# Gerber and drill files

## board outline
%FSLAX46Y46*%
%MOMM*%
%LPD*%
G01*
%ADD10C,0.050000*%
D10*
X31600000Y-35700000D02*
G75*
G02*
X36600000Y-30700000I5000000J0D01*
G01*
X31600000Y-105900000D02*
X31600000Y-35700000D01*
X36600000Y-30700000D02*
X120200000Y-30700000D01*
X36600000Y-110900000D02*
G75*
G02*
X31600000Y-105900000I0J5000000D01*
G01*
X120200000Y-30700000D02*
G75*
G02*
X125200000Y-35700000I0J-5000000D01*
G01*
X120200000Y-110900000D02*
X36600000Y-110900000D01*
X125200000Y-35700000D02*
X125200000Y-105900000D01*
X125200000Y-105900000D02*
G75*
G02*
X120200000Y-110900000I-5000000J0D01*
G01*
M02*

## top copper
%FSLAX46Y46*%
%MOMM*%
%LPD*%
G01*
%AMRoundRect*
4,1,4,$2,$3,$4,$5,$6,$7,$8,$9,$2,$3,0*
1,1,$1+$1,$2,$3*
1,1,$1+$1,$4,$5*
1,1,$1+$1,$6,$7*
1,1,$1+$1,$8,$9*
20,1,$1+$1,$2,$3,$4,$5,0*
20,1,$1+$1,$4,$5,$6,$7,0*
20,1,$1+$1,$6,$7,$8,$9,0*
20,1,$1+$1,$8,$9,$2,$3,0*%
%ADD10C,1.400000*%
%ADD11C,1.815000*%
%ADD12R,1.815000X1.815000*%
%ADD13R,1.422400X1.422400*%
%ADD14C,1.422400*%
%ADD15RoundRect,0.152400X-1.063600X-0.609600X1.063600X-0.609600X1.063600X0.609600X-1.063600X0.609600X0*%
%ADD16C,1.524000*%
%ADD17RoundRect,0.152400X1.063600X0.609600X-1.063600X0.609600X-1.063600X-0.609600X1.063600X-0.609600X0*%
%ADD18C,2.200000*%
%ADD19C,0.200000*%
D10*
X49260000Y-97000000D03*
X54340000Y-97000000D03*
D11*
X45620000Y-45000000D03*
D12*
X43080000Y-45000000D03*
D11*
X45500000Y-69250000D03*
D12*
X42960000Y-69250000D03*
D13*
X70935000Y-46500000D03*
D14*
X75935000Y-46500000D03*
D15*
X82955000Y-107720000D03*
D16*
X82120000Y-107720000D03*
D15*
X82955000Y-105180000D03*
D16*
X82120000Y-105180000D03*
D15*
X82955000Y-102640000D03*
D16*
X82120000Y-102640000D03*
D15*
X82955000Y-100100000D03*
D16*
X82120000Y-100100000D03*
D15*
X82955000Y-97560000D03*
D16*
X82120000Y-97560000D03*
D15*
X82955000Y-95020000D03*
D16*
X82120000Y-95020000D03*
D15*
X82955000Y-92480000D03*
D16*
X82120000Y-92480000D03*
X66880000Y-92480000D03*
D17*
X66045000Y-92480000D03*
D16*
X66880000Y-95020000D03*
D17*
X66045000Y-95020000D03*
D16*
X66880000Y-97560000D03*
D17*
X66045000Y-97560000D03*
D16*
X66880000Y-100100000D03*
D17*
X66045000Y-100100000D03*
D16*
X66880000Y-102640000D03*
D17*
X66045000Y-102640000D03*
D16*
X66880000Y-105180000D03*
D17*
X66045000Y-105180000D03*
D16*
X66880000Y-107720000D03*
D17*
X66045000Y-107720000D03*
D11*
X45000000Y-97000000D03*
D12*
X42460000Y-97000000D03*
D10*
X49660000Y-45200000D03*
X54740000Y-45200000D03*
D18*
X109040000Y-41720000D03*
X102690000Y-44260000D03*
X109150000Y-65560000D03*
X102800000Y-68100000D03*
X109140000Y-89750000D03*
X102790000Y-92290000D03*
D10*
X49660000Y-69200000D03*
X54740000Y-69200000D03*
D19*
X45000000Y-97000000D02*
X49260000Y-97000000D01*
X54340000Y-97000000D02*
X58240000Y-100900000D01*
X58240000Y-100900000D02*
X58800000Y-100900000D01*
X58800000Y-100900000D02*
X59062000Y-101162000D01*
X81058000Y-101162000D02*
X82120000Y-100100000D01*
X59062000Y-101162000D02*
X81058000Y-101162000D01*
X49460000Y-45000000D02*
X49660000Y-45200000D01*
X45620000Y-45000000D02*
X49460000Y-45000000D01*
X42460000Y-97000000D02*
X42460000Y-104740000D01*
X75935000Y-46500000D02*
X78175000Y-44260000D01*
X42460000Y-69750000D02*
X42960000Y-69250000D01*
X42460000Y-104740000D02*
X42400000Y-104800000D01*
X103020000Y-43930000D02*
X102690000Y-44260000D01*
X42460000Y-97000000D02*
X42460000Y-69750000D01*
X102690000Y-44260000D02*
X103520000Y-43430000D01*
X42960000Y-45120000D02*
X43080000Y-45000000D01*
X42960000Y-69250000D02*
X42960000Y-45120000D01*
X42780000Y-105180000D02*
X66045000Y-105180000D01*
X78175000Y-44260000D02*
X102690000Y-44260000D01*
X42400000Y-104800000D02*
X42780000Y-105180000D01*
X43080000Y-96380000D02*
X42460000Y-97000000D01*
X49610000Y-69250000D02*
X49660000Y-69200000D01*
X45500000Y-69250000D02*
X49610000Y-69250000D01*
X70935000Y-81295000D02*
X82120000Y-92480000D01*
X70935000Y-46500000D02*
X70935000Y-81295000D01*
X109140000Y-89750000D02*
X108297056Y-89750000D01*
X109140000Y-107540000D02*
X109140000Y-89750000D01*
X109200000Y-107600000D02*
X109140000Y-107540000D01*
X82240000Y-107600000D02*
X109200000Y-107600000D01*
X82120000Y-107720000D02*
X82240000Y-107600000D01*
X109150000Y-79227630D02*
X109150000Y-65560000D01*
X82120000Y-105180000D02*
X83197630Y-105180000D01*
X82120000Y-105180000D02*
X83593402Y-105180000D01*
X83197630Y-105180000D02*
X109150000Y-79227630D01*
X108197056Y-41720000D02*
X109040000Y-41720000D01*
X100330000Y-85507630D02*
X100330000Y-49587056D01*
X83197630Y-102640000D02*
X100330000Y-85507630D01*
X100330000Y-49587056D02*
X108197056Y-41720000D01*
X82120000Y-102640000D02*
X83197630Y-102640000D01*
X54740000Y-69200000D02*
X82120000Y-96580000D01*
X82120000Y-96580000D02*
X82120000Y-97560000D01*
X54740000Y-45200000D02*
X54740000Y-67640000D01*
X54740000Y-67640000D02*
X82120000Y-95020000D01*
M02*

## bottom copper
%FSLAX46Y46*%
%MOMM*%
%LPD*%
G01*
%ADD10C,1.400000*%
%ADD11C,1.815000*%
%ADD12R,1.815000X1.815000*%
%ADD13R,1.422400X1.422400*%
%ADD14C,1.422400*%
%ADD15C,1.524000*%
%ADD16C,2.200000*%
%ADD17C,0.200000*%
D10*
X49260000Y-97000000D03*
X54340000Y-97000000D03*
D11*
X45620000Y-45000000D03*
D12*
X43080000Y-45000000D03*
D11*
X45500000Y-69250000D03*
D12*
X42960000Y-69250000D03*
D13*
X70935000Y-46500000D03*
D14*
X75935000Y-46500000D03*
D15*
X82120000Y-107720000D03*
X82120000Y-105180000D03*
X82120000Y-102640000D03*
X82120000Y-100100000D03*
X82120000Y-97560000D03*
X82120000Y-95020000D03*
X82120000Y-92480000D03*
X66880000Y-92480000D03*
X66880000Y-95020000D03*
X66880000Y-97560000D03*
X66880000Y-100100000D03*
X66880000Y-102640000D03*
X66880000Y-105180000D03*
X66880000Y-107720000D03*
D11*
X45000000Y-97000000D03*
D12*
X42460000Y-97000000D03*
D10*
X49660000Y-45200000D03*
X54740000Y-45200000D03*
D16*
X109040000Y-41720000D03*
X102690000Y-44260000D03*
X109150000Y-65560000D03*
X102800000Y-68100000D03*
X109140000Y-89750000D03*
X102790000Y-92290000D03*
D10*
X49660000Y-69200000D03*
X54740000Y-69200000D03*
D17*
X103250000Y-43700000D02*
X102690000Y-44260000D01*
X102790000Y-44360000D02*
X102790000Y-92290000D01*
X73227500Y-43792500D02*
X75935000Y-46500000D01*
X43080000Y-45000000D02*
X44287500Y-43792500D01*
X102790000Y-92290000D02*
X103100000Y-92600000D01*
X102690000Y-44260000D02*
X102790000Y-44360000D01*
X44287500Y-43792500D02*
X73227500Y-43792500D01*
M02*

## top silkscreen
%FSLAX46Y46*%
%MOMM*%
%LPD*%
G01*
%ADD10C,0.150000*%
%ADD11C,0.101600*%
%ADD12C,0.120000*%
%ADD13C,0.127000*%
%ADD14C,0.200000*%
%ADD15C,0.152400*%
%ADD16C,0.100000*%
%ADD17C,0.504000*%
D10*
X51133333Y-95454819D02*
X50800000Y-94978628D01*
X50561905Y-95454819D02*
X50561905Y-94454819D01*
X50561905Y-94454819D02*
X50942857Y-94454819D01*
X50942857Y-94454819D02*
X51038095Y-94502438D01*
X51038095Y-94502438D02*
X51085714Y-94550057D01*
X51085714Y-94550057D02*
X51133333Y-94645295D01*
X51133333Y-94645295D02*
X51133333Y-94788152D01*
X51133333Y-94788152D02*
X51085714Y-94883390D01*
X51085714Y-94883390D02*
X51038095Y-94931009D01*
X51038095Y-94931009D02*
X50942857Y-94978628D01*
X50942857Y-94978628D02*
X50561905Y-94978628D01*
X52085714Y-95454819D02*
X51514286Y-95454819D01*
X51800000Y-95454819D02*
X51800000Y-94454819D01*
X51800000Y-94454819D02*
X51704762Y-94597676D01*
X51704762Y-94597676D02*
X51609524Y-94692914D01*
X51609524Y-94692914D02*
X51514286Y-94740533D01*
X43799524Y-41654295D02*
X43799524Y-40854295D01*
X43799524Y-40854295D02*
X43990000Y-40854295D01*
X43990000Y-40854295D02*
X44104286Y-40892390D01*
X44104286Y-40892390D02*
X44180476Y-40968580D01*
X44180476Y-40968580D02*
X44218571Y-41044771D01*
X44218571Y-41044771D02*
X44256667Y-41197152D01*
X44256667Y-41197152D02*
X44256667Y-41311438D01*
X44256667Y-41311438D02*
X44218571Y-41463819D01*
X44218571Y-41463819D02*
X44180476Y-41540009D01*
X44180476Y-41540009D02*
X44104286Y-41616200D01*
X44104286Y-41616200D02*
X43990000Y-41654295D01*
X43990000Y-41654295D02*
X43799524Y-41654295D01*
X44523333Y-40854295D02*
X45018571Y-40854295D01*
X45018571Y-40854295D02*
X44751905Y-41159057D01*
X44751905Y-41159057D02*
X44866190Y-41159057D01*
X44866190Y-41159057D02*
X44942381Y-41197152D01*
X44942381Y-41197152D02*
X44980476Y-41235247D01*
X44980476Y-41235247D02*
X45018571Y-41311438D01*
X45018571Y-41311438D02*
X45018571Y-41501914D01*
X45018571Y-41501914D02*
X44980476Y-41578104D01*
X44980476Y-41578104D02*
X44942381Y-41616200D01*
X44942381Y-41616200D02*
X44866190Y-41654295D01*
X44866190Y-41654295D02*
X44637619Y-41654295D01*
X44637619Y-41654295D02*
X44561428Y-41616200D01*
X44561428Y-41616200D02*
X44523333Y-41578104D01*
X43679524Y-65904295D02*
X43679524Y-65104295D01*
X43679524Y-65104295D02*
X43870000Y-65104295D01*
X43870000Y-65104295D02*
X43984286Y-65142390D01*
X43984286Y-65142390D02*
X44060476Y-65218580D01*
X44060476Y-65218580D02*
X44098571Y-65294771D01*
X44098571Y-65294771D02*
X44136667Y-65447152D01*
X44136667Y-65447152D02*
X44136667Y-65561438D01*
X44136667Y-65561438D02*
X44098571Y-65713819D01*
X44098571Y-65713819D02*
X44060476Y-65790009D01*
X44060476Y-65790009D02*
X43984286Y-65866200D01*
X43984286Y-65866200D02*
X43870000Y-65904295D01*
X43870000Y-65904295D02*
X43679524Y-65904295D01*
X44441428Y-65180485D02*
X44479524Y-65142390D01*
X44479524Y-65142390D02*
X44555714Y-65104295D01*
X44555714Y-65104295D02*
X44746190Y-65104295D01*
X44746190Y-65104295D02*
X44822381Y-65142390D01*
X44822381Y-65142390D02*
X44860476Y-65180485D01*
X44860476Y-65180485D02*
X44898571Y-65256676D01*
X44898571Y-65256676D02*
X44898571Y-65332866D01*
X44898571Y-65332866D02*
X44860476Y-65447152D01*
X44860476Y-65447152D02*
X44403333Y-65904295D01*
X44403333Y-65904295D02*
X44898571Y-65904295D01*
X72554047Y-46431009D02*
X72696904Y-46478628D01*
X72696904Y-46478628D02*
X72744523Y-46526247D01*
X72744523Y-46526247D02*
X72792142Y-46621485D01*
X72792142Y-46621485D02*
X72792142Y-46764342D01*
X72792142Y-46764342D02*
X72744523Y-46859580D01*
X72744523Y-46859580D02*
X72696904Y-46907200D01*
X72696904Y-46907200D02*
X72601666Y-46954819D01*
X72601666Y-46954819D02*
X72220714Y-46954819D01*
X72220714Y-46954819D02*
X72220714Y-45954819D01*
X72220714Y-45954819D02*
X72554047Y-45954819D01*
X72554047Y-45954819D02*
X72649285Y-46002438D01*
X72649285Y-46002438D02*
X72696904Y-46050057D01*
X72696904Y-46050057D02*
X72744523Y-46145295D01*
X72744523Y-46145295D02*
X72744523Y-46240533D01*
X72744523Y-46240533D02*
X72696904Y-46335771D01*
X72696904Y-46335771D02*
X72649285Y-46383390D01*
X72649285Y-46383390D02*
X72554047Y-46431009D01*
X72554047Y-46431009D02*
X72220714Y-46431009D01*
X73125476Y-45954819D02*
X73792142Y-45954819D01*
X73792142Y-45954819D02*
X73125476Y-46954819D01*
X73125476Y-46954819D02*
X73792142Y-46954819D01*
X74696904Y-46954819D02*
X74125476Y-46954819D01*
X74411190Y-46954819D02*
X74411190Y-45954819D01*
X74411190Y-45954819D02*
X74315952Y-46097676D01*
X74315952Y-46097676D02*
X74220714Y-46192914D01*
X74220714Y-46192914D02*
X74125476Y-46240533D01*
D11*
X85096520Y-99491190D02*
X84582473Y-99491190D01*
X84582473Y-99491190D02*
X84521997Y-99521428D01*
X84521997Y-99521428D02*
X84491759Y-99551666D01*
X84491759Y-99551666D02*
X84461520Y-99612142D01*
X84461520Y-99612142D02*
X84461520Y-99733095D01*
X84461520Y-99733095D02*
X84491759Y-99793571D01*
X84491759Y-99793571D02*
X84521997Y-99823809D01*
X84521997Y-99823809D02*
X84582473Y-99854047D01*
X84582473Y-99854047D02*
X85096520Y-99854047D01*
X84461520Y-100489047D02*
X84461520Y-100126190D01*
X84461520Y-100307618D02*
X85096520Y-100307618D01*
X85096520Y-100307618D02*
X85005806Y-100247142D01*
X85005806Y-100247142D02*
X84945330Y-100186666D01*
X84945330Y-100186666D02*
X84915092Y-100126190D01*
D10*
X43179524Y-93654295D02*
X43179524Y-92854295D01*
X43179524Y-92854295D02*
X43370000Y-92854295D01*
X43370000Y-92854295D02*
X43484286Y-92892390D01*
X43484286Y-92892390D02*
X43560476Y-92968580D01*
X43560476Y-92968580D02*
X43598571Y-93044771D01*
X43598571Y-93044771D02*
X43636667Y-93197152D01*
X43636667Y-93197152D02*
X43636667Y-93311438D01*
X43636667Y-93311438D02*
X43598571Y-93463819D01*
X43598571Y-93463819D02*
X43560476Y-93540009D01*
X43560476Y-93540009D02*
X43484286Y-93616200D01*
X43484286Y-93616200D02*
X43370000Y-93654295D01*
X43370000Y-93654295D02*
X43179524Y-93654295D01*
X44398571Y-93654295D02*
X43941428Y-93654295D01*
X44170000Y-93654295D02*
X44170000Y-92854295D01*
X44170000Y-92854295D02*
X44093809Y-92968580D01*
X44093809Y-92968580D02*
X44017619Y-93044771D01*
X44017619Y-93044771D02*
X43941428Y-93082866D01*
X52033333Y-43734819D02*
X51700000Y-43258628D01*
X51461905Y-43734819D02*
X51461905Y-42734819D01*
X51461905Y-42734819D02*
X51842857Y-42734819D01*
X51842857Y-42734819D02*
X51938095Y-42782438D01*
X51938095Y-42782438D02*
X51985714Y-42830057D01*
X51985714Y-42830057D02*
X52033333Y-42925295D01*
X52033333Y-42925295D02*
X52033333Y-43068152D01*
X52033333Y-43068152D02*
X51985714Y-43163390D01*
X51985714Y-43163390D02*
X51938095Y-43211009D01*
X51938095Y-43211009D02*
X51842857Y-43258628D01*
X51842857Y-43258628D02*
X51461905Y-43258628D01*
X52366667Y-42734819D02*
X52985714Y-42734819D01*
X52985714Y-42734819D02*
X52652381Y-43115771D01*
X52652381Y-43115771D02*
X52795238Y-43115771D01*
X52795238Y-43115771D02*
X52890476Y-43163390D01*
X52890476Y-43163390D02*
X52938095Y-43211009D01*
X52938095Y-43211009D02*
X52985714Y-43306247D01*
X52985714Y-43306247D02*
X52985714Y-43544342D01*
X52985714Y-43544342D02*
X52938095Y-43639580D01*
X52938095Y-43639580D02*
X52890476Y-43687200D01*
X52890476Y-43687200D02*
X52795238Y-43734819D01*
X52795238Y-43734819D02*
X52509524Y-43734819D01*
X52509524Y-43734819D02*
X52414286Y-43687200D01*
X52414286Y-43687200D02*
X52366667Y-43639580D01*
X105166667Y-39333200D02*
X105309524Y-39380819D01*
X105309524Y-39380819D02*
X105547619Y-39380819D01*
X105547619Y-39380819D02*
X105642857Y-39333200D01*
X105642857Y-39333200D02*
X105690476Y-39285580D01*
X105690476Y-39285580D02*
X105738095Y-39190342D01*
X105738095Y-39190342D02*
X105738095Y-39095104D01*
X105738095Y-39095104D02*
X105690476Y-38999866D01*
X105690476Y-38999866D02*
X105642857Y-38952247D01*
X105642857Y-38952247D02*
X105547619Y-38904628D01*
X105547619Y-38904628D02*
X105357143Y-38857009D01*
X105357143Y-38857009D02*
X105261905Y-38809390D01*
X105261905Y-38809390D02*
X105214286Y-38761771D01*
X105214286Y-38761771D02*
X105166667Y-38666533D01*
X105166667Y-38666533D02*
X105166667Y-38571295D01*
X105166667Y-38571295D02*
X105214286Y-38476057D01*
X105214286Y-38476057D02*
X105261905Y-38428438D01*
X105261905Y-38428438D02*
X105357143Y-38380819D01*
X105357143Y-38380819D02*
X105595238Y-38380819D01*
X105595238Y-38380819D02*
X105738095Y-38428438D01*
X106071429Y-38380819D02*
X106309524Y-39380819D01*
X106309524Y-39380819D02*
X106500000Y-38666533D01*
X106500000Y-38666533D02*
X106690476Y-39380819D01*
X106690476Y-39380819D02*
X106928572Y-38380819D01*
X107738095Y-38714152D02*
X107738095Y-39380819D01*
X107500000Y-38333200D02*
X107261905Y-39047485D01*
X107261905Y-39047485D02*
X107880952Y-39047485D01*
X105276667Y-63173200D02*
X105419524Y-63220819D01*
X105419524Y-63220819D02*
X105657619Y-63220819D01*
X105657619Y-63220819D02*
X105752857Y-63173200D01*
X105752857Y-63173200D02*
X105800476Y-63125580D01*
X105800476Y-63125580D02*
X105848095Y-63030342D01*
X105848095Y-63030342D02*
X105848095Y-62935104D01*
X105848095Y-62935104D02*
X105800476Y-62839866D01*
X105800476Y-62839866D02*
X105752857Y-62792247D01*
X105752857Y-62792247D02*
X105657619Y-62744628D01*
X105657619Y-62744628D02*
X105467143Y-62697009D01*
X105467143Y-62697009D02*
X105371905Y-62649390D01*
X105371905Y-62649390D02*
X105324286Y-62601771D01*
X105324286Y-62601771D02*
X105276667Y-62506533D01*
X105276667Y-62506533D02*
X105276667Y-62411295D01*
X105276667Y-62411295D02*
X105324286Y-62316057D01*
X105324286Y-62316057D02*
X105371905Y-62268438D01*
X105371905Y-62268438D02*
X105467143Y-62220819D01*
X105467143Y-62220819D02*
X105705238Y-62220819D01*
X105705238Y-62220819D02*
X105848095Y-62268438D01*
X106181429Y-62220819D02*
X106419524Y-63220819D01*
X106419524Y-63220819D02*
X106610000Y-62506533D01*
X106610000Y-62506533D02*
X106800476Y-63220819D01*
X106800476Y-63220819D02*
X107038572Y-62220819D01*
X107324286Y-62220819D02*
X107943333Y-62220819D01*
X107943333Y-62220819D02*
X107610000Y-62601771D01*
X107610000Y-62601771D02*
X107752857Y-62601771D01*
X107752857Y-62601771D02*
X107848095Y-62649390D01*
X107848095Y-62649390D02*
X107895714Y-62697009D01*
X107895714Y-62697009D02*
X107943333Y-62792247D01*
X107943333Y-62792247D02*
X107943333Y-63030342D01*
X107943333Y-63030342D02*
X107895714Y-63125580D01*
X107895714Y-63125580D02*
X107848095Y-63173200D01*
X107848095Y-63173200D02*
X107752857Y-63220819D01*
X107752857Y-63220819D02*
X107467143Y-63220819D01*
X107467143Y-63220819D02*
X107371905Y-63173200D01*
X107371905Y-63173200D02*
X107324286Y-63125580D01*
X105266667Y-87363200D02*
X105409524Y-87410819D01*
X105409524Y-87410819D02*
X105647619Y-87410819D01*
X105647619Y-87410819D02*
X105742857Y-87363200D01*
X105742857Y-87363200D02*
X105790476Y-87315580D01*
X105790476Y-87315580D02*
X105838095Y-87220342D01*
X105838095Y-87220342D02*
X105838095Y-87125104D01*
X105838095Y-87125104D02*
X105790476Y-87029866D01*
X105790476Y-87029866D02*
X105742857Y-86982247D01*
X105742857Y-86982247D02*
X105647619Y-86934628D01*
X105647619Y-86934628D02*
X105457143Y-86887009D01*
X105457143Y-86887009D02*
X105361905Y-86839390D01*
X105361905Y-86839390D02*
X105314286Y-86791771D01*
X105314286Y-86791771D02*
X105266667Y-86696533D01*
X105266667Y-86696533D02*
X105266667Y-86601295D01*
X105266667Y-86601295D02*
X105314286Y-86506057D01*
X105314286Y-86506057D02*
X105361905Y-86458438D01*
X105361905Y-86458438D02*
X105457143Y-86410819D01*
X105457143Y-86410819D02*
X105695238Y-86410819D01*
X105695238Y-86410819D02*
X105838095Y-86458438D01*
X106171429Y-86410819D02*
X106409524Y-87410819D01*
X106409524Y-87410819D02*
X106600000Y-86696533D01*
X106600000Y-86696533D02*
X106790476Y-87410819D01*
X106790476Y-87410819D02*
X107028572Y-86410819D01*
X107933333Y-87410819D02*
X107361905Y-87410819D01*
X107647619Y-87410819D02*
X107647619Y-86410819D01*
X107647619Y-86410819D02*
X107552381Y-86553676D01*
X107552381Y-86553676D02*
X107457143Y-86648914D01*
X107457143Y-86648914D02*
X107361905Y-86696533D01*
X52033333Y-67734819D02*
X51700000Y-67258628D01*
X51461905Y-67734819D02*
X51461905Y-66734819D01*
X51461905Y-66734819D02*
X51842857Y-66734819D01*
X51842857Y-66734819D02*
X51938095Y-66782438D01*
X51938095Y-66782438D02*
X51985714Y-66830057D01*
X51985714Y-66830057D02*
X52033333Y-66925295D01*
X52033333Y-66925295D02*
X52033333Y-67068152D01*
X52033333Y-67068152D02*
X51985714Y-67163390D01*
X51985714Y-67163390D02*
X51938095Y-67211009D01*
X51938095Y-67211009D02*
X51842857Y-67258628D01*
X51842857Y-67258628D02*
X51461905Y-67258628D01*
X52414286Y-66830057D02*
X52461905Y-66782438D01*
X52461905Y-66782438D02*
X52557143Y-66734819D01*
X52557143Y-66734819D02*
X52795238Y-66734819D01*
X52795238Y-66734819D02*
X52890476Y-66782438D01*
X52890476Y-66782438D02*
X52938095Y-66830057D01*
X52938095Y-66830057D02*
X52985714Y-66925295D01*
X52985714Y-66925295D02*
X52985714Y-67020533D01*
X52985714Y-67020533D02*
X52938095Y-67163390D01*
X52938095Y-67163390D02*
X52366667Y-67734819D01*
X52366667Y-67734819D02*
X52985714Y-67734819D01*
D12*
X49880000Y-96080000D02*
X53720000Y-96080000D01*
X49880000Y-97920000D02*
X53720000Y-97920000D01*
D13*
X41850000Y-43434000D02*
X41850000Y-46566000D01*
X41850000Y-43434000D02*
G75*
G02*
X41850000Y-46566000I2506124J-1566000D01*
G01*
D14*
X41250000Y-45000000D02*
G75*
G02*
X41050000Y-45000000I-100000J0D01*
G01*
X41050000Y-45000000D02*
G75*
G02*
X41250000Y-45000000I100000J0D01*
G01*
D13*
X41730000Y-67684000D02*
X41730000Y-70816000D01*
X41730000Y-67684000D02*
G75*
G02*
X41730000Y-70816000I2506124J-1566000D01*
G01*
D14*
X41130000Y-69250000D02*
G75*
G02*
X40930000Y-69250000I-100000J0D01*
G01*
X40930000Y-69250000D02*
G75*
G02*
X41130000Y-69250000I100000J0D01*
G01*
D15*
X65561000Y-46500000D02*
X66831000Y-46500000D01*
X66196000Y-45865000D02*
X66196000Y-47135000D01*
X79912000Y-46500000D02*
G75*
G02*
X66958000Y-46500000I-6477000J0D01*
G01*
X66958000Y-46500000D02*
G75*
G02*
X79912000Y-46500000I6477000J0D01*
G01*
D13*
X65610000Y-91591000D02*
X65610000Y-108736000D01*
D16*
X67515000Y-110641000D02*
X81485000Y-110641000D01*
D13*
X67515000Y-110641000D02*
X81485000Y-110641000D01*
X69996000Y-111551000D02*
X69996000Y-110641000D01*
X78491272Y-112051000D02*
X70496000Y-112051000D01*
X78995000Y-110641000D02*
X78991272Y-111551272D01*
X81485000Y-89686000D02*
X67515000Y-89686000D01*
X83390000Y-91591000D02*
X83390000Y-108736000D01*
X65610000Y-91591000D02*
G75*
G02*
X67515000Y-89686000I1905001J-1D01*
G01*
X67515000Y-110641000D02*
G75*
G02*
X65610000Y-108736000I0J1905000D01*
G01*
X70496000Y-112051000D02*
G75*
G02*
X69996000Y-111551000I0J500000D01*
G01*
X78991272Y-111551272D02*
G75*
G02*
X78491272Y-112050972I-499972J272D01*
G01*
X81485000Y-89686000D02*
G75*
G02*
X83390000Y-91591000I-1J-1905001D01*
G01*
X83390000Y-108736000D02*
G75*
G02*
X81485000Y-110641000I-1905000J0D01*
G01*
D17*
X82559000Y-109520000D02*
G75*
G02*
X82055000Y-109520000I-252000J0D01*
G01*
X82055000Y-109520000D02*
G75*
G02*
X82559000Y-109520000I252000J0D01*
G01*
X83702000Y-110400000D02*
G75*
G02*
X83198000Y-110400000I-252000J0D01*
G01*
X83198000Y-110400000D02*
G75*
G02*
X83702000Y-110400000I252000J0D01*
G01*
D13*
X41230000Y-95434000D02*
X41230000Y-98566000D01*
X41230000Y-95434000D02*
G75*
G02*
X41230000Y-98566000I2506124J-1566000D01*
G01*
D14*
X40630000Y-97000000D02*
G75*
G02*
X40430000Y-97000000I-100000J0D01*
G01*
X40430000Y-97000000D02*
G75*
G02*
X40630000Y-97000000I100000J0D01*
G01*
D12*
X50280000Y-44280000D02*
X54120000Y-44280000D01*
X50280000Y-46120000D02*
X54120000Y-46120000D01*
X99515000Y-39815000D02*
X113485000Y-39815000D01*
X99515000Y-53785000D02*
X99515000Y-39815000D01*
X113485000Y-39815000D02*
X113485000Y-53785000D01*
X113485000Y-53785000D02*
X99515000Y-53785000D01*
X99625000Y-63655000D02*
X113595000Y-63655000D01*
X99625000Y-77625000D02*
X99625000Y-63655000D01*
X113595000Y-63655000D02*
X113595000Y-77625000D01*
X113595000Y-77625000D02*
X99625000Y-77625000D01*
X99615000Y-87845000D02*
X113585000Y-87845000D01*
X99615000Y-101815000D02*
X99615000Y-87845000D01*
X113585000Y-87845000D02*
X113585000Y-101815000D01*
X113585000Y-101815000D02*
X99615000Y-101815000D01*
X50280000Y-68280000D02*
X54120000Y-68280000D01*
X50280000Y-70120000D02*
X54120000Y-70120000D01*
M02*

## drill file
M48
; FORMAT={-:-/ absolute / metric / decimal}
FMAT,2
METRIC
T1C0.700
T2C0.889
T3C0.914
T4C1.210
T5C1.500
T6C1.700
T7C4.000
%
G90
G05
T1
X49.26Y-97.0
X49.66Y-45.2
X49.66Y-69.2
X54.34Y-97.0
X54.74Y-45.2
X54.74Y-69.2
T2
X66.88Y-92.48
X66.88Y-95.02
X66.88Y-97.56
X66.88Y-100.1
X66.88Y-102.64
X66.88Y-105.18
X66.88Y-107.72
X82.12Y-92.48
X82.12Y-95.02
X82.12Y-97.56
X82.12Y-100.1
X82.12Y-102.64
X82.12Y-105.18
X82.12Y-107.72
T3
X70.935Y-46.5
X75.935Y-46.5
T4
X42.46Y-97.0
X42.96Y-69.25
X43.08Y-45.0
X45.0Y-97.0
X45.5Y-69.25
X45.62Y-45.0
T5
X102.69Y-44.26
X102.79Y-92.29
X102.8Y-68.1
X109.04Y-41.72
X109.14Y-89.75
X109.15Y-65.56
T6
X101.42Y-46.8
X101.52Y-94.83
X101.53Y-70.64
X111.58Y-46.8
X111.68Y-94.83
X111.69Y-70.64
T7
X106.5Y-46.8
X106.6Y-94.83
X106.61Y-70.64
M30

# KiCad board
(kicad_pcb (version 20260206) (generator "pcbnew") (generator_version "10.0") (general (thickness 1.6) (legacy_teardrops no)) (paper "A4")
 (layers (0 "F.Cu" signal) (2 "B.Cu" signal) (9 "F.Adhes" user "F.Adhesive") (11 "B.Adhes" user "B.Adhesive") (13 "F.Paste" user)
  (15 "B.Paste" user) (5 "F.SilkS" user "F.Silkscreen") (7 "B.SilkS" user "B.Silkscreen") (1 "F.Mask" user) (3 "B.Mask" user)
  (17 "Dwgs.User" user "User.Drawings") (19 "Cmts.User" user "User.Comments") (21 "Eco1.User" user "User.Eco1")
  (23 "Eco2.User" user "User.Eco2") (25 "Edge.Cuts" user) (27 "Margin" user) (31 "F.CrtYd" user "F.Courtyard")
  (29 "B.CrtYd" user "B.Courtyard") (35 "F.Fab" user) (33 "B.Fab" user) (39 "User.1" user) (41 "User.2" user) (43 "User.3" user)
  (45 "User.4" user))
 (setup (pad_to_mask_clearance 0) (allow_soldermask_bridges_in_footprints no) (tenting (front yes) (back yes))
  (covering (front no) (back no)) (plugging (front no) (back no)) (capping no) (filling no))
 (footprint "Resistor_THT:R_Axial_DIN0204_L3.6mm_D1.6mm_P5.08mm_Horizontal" (layer "F.Cu") (at 49.26 97)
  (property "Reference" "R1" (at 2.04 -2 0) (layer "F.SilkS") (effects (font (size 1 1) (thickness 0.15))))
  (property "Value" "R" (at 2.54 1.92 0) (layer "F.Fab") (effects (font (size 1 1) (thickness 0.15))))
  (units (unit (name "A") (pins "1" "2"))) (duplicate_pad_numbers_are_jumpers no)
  (fp_line (start 0.62 -0.92) (end 4.46 -0.92) (stroke (width 0.12) (type solid)) (layer "F.SilkS"))
  (fp_line (start 0.62 0.92) (end 4.46 0.92) (stroke (width 0.12) (type solid)) (layer "F.SilkS"))
  (pad "1" thru_hole circle (at 0 0) (size 1.4 1.4) (drill 0.7) (layers "*.Cu" "*.Mask") (remove_unused_layers no) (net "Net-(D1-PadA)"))
  (pad "2" thru_hole circle (at 5.08 0) (size 1.4 1.4) (drill 0.7) (layers "*.Cu" "*.Mask") (remove_unused_layers no) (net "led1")))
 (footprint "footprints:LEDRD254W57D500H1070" (layer "F.Cu") (at 44.35 45)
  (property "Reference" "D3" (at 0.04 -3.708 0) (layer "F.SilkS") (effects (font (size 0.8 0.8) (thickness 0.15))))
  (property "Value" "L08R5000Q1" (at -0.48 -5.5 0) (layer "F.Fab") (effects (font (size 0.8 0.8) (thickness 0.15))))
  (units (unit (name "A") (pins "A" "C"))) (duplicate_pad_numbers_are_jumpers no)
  (fp_line (start -2.5 -1.566) (end -2.5 1.566) (stroke (width 0.127) (type solid)) (layer "F.SilkS"))
  (fp_arc (start -2.5 -1.566) (mid 2.961291 0) (end -2.5 1.566) (stroke (width 0.127) (type solid)) (layer "F.SilkS"))
  (fp_circle (center -3.2 0) (end -3.1 0) (stroke (width 0.2) (type solid)) (fill no) (layer "F.SilkS"))
  (pad "A" thru_hole circle (at 1.27 0) (size 1.815 1.815) (drill 1.21) (layers "*.Cu" "*.Mask") (remove_unused_layers no)
   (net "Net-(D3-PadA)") (solder_mask_margin 0.102))
  (pad "C" thru_hole rect (at -1.27 0) (size 1.815 1.815) (drill 1.21) (layers "*.Cu" "*.Mask") (remove_unused_layers no) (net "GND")
   (solder_mask_margin 0.102)))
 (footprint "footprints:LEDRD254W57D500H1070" (layer "F.Cu") (at 44.23 69.25)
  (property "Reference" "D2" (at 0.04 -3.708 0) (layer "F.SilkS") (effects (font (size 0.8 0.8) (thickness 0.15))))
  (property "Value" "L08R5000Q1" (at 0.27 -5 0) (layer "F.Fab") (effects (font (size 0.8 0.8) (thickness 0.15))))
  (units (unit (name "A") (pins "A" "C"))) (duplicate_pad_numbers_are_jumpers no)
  (fp_line (start -2.5 -1.566) (end -2.5 1.566) (stroke (width 0.127) (type solid)) (layer "F.SilkS"))
  (fp_arc (start -2.5 -1.566) (mid 2.961291 0) (end -2.5 1.566) (stroke (width 0.127) (type solid)) (layer "F.SilkS"))
  (fp_circle (center -3.2 0) (end -3.1 0) (stroke (width 0.2) (type solid)) (fill no) (layer "F.SilkS"))
  (pad "A" thru_hole circle (at 1.27 0) (size 1.815 1.815) (drill 1.21) (layers "*.Cu" "*.Mask") (remove_unused_layers no)
   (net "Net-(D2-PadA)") (solder_mask_margin 0.102))
  (pad "C" thru_hole rect (at -1.27 0) (size 1.815 1.815) (drill 1.21) (layers "*.Cu" "*.Mask") (remove_unused_layers no) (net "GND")
   (solder_mask_margin 0.102)))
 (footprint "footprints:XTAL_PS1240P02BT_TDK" (layer "F.Cu") (at 70.935 46.5)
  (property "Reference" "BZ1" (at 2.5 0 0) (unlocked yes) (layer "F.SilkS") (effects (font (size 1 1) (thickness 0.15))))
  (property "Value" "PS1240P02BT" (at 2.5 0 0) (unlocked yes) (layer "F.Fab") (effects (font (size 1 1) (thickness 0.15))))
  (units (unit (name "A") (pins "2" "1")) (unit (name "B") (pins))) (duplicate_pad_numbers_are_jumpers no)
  (fp_line (start -5.374 0) (end -4.104 0) (stroke (width 0.1524) (type solid)) (layer "F.SilkS"))
  (fp_line (start -4.739 -0.635) (end -4.739 0.635) (stroke (width 0.1524) (type solid)) (layer "F.SilkS"))
  (fp_circle (center 2.5 0) (end 8.977 0) (stroke (width 0.1524) (type solid)) (fill no) (layer "F.SilkS"))
  (pad "1" thru_hole rect (at 0 0) (size 1.4224 1.4224) (drill 0.9144) (layers "*.Cu" "*.Mask") (remove_unused_layers no) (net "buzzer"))
  (pad "2" thru_hole circle (at 5 0) (size 1.4224 1.4224) (drill 0.9144) (layers "*.Cu" "*.Mask") (remove_unused_layers no) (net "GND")))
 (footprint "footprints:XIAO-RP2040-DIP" (layer "F.Cu") (at 74.5 100.1 -90)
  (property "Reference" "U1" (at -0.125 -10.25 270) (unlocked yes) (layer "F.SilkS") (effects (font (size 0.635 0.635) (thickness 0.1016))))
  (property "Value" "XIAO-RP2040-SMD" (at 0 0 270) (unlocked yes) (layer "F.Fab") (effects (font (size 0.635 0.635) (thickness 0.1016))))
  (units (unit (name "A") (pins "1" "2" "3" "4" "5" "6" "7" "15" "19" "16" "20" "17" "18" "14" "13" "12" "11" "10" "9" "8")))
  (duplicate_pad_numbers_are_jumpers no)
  (fp_line (start -8.509 8.89) (end 8.636 8.89) (stroke (width 0.127) (type solid)) (layer "F.SilkS"))
  (fp_line (start 10.541 6.985) (end 10.541 -6.985) (stroke (width 0.1) (type solid)) (layer "F.SilkS"))
  (fp_line (start 10.541 6.985) (end 10.541 -6.985) (stroke (width 0.127) (type solid)) (layer "F.SilkS"))
  (fp_line (start 11.451 4.504) (end 10.541 4.504) (stroke (width 0.127) (type solid)) (layer "F.SilkS"))
  (fp_line (start 11.951 -3.991272) (end 11.951 4.004) (stroke (width 0.127) (type solid)) (layer "F.SilkS"))
  (fp_line (start 10.541 -4.495) (end 11.451272 -4.491272) (stroke (width 0.127) (type solid)) (layer "F.SilkS"))
  (fp_line (start -10.414 -6.985) (end -10.414 6.985) (stroke (width 0.127) (type solid)) (layer "F.SilkS"))
  (fp_line (start -8.509 -8.89) (end 8.636 -8.89) (stroke (width 0.127) (type solid)) (layer "F.SilkS"))
  (fp_arc (start -8.509 8.89) (mid -9.856038 8.332038) (end -10.414 6.985) (stroke (width 0.127) (type solid)) (layer "F.SilkS"))
  (fp_arc (start 10.541 6.985) (mid 9.983038 8.332038) (end 8.636 8.89) (stroke (width 0.127) (type solid)) (layer "F.SilkS"))
  (fp_arc (start 11.951 4.004) (mid 11.804553 4.357553) (end 11.451 4.504) (stroke (width 0.127) (type default)) (layer "F.SilkS"))
  (fp_arc (start 11.451272 -4.491272) (mid 11.804644 -4.344724) (end 11.951 -3.991272) (stroke (width 0.127) (type default))
   (layer "F.SilkS"))
  (fp_arc (start -10.414 -6.985) (mid -9.856038 -8.332038) (end -8.509 -8.89) (stroke (width 0.127) (type solid)) (layer "F.SilkS"))
  (fp_arc (start 8.636 -8.89) (mid 9.983038 -8.332038) (end 10.541 -6.985) (stroke (width 0.127) (type solid)) (layer "F.SilkS"))
  (fp_circle (center 9.42 -7.807) (end 9.674 -7.807) (stroke (width 0.5) (type solid)) (fill yes) (layer "F.SilkS"))
  (fp_circle (center 10.3 -8.95) (end 10.554 -8.95) (stroke (width 0.5) (type solid)) (fill yes) (layer "F.SilkS"))
  (pad "1" smd roundrect (at 7.62 -8.455) (size 2.432 1.524) (layers "F.Cu" "F.Mask") (roundrect_rratio 0.1) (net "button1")
   (thermal_bridge_angle 45))
  (pad "1" thru_hole circle (at 7.62 -7.62) (size 1.524 1.524) (drill 0.889) (layers "*.Cu" "*.Mask") (remove_unused_layers no)
   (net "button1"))
  (pad "2" smd roundrect (at 5.08 -8.455) (size 2.432 1.524) (layers "F.Cu" "F.Mask") (roundrect_rratio 0.1) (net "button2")
   (thermal_bridge_angle 45))
  (pad "2" thru_hole circle (at 5.08 -7.62) (size 1.524 1.524) (drill 0.889) (layers "*.Cu" "*.Mask") (remove_unused_layers no)
   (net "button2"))
  (pad "3" smd roundrect (at 2.54 -8.455) (size 2.432 1.524) (layers "F.Cu" "F.Mask") (roundrect_rratio 0.1) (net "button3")
   (thermal_bridge_angle 45))
  (pad "3" thru_hole circle (at 2.54 -7.62) (size 1.524 1.524) (drill 0.889) (layers "*.Cu" "*.Mask") (remove_unused_layers no)
   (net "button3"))
  (pad "4" smd roundrect (at 0 -8.455) (size 2.432 1.524) (layers "F.Cu" "F.Mask") (roundrect_rratio 0.1) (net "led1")
   (thermal_bridge_angle 45))
  (pad "4" thru_hole circle (at 0 -7.62) (size 1.524 1.524) (drill 0.889) (layers "*.Cu" "*.Mask") (remove_unused_layers no) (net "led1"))
  (pad "5" smd roundrect (at -2.54 -8.455) (size 2.432 1.524) (layers "F.Cu" "F.Mask") (roundrect_rratio 0.1) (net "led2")
   (thermal_bridge_angle 45))
  (pad "5" thru_hole circle (at -2.54 -7.62) (size 1.524 1.524) (drill 0.889) (layers "*.Cu" "*.Mask") (remove_unused_layers no)
   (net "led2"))
  (pad "6" smd roundrect (at -5.08 -8.455) (size 2.432 1.524) (layers "F.Cu" "F.Mask") (roundrect_rratio 0.1) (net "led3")
   (thermal_bridge_angle 45))
  (pad "6" thru_hole circle (at -5.08 -7.62) (size 1.524 1.524) (drill 0.889) (layers "*.Cu" "*.Mask") (remove_unused_layers no)
   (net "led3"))
  (pad "7" smd roundrect (at -7.62 -8.455) (size 2.432 1.524) (layers "F.Cu" "F.Mask") (roundrect_rratio 0.1) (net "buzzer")
   (thermal_bridge_angle 45))
  (pad "7" thru_hole circle (at -7.62 -7.62) (size 1.524 1.524) (drill 0.889) (layers "*.Cu" "*.Mask") (remove_unused_layers no)
   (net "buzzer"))
  (pad "8" thru_hole circle (at -7.62 7.62 180) (size 1.524 1.524) (drill 0.889) (layers "*.Cu" "*.Mask") (remove_unused_layers no)
   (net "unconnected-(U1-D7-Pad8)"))
  (pad "8" smd roundrect (at -7.62 8.455 180) (size 2.432 1.524) (layers "F.Cu" "F.Mask") (roundrect_rratio 0.1)
   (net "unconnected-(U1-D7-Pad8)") (thermal_bridge_angle 45))
  (pad "9" thru_hole circle (at -5.08 7.62 180) (size 1.524 1.524) (drill 0.889) (layers "*.Cu" "*.Mask") (remove_unused_layers no)
   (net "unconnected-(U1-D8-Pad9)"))
  (pad "9" smd roundrect (at -5.08 8.455 180) (size 2.432 1.524) (layers "F.Cu" "F.Mask") (roundrect_rratio 0.1)
   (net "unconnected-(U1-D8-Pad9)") (thermal_bridge_angle 45))
  (pad "10" thru_hole circle (at -2.54 7.62 180) (size 1.524 1.524) (drill 0.889) (layers "*.Cu" "*.Mask") (remove_unused_layers no)
   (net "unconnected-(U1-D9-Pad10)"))
  (pad "10" smd roundrect (at -2.54 8.455 180) (size 2.432 1.524) (layers "F.Cu" "F.Mask") (roundrect_rratio 0.1)
   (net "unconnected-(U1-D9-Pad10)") (thermal_bridge_angle 45))
  (pad "11" thru_hole circle (at 0 7.62 180) (size 1.524 1.524) (drill 0.889) (layers "*.Cu" "*.Mask") (remove_unused_layers no)
   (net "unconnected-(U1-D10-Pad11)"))
  (pad "11" smd roundrect (at 0 8.455 180) (size 2.432 1.524) (layers "F.Cu" "F.Mask") (roundrect_rratio 0.1)
   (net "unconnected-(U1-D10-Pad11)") (thermal_bridge_angle 45))
  (pad "12" thru_hole circle (at 2.54 7.62 180) (size 1.524 1.524) (drill 0.889) (layers "*.Cu" "*.Mask") (remove_unused_layers no)
   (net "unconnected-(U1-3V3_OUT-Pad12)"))
  (pad "12" smd roundrect (at 2.54 8.455 180) (size 2.432 1.524) (layers "F.Cu" "F.Mask") (roundrect_rratio 0.1)
   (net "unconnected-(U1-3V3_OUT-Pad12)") (thermal_bridge_angle 45))
  (pad "13" thru_hole circle (at 5.08 7.62 180) (size 1.524 1.524) (drill 0.889) (layers "*.Cu" "*.Mask") (remove_unused_layers no)
   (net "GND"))
  (pad "13" smd roundrect (at 5.08 8.455 180) (size 2.432 1.524) (layers "F.Cu" "F.Mask") (roundrect_rratio 0.1) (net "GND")
   (thermal_bridge_angle 45))
  (pad "14" thru_hole circle (at 7.62 7.62 180) (size 1.524 1.524) (drill 0.889) (layers "*.Cu" "*.Mask") (remove_unused_layers no)
   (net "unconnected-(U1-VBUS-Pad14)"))
  (pad "14" smd roundrect (at 7.62 8.455 180) (size 2.432 1.524) (layers "F.Cu" "F.Mask") (roundrect_rratio 0.1)
   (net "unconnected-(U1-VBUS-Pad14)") (thermal_bridge_angle 45)))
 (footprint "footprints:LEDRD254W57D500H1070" (layer "F.Cu") (at 43.73 97)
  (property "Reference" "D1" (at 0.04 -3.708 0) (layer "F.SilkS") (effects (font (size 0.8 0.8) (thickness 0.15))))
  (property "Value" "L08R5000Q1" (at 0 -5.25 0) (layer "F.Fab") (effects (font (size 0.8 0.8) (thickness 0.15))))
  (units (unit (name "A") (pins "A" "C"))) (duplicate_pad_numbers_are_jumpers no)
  (fp_line (start -2.5 -1.566) (end -2.5 1.566) (stroke (width 0.127) (type solid)) (layer "F.SilkS"))
  (fp_arc (start -2.5 -1.566) (mid 2.961291 0) (end -2.5 1.566) (stroke (width 0.127) (type solid)) (layer "F.SilkS"))
  (fp_circle (center -3.2 0) (end -3.1 0) (stroke (width 0.2) (type solid)) (fill no) (layer "F.SilkS"))
  (pad "A" thru_hole circle (at 1.27 0) (size 1.815 1.815) (drill 1.21) (layers "*.Cu" "*.Mask") (remove_unused_layers no)
   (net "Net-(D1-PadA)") (solder_mask_margin 0.102))
  (pad "C" thru_hole rect (at -1.27 0) (size 1.815 1.815) (drill 1.21) (layers "*.Cu" "*.Mask") (remove_unused_layers no) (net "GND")
   (solder_mask_margin 0.102)))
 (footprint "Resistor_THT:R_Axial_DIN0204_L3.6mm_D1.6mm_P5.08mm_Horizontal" (layer "F.Cu") (at 49.66 45.2)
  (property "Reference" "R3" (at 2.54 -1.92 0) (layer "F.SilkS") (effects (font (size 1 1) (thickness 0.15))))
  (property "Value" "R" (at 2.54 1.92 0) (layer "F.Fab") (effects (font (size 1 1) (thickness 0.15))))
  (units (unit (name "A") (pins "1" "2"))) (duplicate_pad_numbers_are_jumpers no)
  (fp_line (start 0.62 -0.92) (end 4.46 -0.92) (stroke (width 0.12) (type solid)) (layer "F.SilkS"))
  (fp_line (start 0.62 0.92) (end 4.46 0.92) (stroke (width 0.12) (type solid)) (layer "F.SilkS"))
  (pad "1" thru_hole circle (at 0 0) (size 1.4 1.4) (drill 0.7) (layers "*.Cu" "*.Mask") (remove_unused_layers no) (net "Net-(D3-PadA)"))
  (pad "2" thru_hole circle (at 5.08 0) (size 1.4 1.4) (drill 0.7) (layers "*.Cu" "*.Mask") (remove_unused_layers no) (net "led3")))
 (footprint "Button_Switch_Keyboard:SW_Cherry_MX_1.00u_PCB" (layer "F.Cu") (at 109.04 41.72)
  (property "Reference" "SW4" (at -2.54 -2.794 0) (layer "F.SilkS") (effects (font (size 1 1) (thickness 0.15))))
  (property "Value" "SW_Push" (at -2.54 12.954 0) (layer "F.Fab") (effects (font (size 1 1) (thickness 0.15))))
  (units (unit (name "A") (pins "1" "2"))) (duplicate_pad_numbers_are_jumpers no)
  (fp_line (start -9.525 -1.905) (end 4.445 -1.905) (stroke (width 0.12) (type solid)) (layer "F.SilkS"))
  (fp_line (start -9.525 12.065) (end -9.525 -1.905) (stroke (width 0.12) (type solid)) (layer "F.SilkS"))
  (fp_line (start 4.445 -1.905) (end 4.445 12.065) (stroke (width 0.12) (type solid)) (layer "F.SilkS"))
  (fp_line (start 4.445 12.065) (end -9.525 12.065) (stroke (width 0.12) (type solid)) (layer "F.SilkS"))
  (pad "" np_thru_hole circle (at -7.62 5.08) (size 1.7 1.7) (drill 1.7) (layers "*.Cu" "*.Mask"))
  (pad "" np_thru_hole circle (at -2.54 5.08) (size 4 4) (drill 4) (layers "*.Cu" "*.Mask"))
  (pad "" np_thru_hole circle (at 2.54 5.08) (size 1.7 1.7) (drill 1.7) (layers "*.Cu" "*.Mask"))
  (pad "1" thru_hole circle (at 0 0) (size 2.2 2.2) (drill 1.5) (layers "*.Cu" "*.Mask") (remove_unused_layers no) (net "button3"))
  (pad "2" thru_hole circle (at -6.35 2.54) (size 2.2 2.2) (drill 1.5) (layers "*.Cu" "*.Mask") (remove_unused_layers no) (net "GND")))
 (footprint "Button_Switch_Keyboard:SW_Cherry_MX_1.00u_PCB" (layer "F.Cu") (at 109.15 65.56)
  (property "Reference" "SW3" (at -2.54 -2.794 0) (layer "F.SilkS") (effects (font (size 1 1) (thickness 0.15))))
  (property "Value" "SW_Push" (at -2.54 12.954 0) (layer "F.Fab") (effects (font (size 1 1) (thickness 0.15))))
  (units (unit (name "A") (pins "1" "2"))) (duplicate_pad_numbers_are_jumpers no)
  (fp_line (start -9.525 -1.905) (end 4.445 -1.905) (stroke (width 0.12) (type solid)) (layer "F.SilkS"))
  (fp_line (start -9.525 12.065) (end -9.525 -1.905) (stroke (width 0.12) (type solid)) (layer "F.SilkS"))
  (fp_line (start 4.445 -1.905) (end 4.445 12.065) (stroke (width 0.12) (type solid)) (layer "F.SilkS"))
  (fp_line (start 4.445 12.065) (end -9.525 12.065) (stroke (width 0.12) (type solid)) (layer "F.SilkS"))
  (pad "" np_thru_hole circle (at -7.62 5.08) (size 1.7 1.7) (drill 1.7) (layers "*.Cu" "*.Mask"))
  (pad "" np_thru_hole circle (at -2.54 5.08) (size 4 4) (drill 4) (layers "*.Cu" "*.Mask"))
  (pad "" np_thru_hole circle (at 2.54 5.08) (size 1.7 1.7) (drill 1.7) (layers "*.Cu" "*.Mask"))
  (pad "1" thru_hole circle (at 0 0) (size 2.2 2.2) (drill 1.5) (layers "*.Cu" "*.Mask") (remove_unused_layers no) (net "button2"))
  (pad "2" thru_hole circle (at -6.35 2.54) (size 2.2 2.2) (drill 1.5) (layers "*.Cu" "*.Mask") (remove_unused_layers no) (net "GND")))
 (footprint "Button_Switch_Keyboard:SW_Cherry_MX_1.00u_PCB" (layer "F.Cu") (at 109.14 89.75)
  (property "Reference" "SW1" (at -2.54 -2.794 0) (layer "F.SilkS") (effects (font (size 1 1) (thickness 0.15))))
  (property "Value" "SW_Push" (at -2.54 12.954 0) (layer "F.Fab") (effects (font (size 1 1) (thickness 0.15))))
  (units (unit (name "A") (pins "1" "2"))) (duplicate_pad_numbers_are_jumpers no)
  (fp_line (start -9.525 -1.905) (end 4.445 -1.905) (stroke (width 0.12) (type solid)) (layer "F.SilkS"))
  (fp_line (start -9.525 12.065) (end -9.525 -1.905) (stroke (width 0.12) (type solid)) (layer "F.SilkS"))
  (fp_line (start 4.445 -1.905) (end 4.445 12.065) (stroke (width 0.12) (type solid)) (layer "F.SilkS"))
  (fp_line (start 4.445 12.065) (end -9.525 12.065) (stroke (width 0.12) (type solid)) (layer "F.SilkS"))
  (pad "" np_thru_hole circle (at -7.62 5.08) (size 1.7 1.7) (drill 1.7) (layers "*.Cu" "*.Mask"))
  (pad "" np_thru_hole circle (at -2.54 5.08) (size 4 4) (drill 4) (layers "*.Cu" "*.Mask"))
  (pad "" np_thru_hole circle (at 2.54 5.08) (size 1.7 1.7) (drill 1.7) (layers "*.Cu" "*.Mask"))
  (pad "1" thru_hole circle (at 0 0) (size 2.2 2.2) (drill 1.5) (layers "*.Cu" "*.Mask") (remove_unused_layers no) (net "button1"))
  (pad "2" thru_hole circle (at -6.35 2.54) (size 2.2 2.2) (drill 1.5) (layers "*.Cu" "*.Mask") (remove_unused_layers no) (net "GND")))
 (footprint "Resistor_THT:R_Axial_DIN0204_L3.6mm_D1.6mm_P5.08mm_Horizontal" (layer "F.Cu") (at 49.66 69.2)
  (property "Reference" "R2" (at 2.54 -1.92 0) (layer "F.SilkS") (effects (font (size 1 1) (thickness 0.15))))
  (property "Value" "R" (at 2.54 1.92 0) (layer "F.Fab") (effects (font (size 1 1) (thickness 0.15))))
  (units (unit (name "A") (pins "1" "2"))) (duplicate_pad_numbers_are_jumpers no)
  (fp_line (start 0.62 -0.92) (end 4.46 -0.92) (stroke (width 0.12) (type solid)) (layer "F.SilkS"))
  (fp_line (start 0.62 0.92) (end 4.46 0.92) (stroke (width 0.12) (type solid)) (layer "F.SilkS"))
  (pad "1" thru_hole circle (at 0 0) (size 1.4 1.4) (drill 0.7) (layers "*.Cu" "*.Mask") (remove_unused_layers no) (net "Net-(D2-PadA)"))
  (pad "2" thru_hole circle (at 5.08 0) (size 1.4 1.4) (drill 0.7) (layers "*.Cu" "*.Mask") (remove_unused_layers no) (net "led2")))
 (gr_arc (start 31.6 35.7) (mid 33.064466 32.164466) (end 36.6 30.7) (stroke (width 0.05) (type default)) (layer "Edge.Cuts"))
 (gr_line (start 31.6 105.9) (end 31.6 35.7) (stroke (width 0.05) (type default)) (layer "Edge.Cuts"))
 (gr_line (start 36.6 30.7) (end 120.2 30.7) (stroke (width 0.05) (type default)) (layer "Edge.Cuts"))
 (gr_arc (start 36.6 110.9) (mid 33.064466 109.435534) (end 31.6 105.9) (stroke (width 0.05) (type default)) (layer "Edge.Cuts"))
 (gr_arc (start 120.2 30.7) (mid 123.735534 32.164466) (end 125.2 35.7) (stroke (width 0.05) (type default)) (layer "Edge.Cuts"))
 (gr_line (start 120.2 110.9) (end 36.6 110.9) (stroke (width 0.05) (type default)) (layer "Edge.Cuts"))
 (gr_line (start 125.2 35.7) (end 125.2 105.9) (stroke (width 0.05) (type default)) (layer "Edge.Cuts"))
 (gr_arc (start 125.2 105.9) (mid 123.735534 109.435534) (end 120.2 110.9) (stroke (width 0.05) (type default)) (layer "Edge.Cuts"))
 (segment (start 45 97) (end 49.26 97) (width 0.2) (layer "F.Cu") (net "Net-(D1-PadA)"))
 (segment (start 54.34 97) (end 58.24 100.9) (width 0.2) (layer "F.Cu") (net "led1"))
 (segment (start 58.24 100.9) (end 58.8 100.9) (width 0.2) (layer "F.Cu") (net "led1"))
 (segment (start 58.8 100.9) (end 59.062 101.162) (width 0.2) (layer "F.Cu") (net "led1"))
 (segment (start 81.058 101.162) (end 82.12 100.1) (width 0.2) (layer "F.Cu") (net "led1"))
 (segment (start 59.062 101.162) (end 81.058 101.162) (width 0.2) (layer "F.Cu") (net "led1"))
 (segment (start 49.46 45) (end 49.66 45.2) (width 0.2) (layer "F.Cu") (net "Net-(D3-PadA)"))
 (segment (start 45.62 45) (end 49.46 45) (width 0.2) (layer "F.Cu") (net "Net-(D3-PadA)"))
 (segment (start 42.46 97) (end 42.46 104.74) (width 0.2) (layer "F.Cu") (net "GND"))
 (segment (start 75.935 46.5) (end 78.175 44.26) (width 0.2) (layer "F.Cu") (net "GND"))
 (segment (start 42.46 69.75) (end 42.96 69.25) (width 0.2) (layer "F.Cu") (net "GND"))
 (segment (start 42.46 104.74) (end 42.4 104.8) (width 0.2) (layer "F.Cu") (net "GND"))
 (segment (start 103.02 43.93) (end 102.69 44.26) (width 0.2) (layer "F.Cu") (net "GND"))
 (segment (start 42.46 97) (end 42.46 69.75) (width 0.2) (layer "F.Cu") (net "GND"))
 (segment (start 102.69 44.26) (end 103.52 43.43) (width 0.2) (layer "F.Cu") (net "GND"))
 (segment (start 42.96 45.12) (end 43.08 45) (width 0.2) (layer "F.Cu") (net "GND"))
 (segment (start 42.96 69.25) (end 42.96 45.12) (width 0.2) (layer "F.Cu") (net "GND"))
 (segment (start 42.78 105.18) (end 66.045 105.18) (width 0.2) (layer "F.Cu") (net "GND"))
 (segment (start 78.175 44.26) (end 102.69 44.26) (width 0.2) (layer "F.Cu") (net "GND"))
 (segment (start 42.4 104.8) (end 42.78 105.18) (width 0.2) (layer "F.Cu") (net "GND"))
 (segment (start 43.08 96.38) (end 42.46 97) (width 0.2) (layer "F.Cu") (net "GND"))
 (segment (start 103.25 43.7) (end 102.69 44.26) (width 0.2) (layer "B.Cu") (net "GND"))
 (segment (start 102.79 44.36) (end 102.79 92.29) (width 0.2) (layer "B.Cu") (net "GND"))
 (segment (start 73.2275 43.7925) (end 75.935 46.5) (width 0.2) (layer "B.Cu") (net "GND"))
 (segment (start 43.08 45) (end 44.2875 43.7925) (width 0.2) (layer "B.Cu") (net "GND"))
 (segment (start 102.79 92.29) (end 103.1 92.6) (width 0.2) (layer "B.Cu") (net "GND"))
 (segment (start 102.69 44.26) (end 102.79 44.36) (width 0.2) (layer "B.Cu") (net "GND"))
 (segment (start 44.2875 43.7925) (end 73.2275 43.7925) (width 0.2) (layer "B.Cu") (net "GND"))
 (segment (start 49.61 69.25) (end 49.66 69.2) (width 0.2) (layer "F.Cu") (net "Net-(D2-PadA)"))
 (segment (start 45.5 69.25) (end 49.61 69.25) (width 0.2) (layer "F.Cu") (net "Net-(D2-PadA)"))
 (segment (start 70.935 81.295) (end 82.12 92.48) (width 0.2) (layer "F.Cu") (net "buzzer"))
 (segment (start 70.935 46.5) (end 70.935 81.295) (width 0.2) (layer "F.Cu") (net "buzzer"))
 (segment (start 109.14 89.75) (end 108.297056 89.75) (width 0.2) (layer "F.Cu") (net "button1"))
 (segment (start 109.14 107.54) (end 109.14 89.75) (width 0.2) (layer "F.Cu") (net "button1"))
 (segment (start 109.2 107.6) (end 109.14 107.54) (width 0.2) (layer "F.Cu") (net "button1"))
 (segment (start 82.24 107.6) (end 109.2 107.6) (width 0.2) (layer "F.Cu") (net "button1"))
 (segment (start 82.12 107.72) (end 82.24 107.6) (width 0.2) (layer "F.Cu") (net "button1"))
 (segment (start 109.15 79.22763) (end 109.15 65.56) (width 0.2) (layer "F.Cu") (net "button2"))
 (segment (start 82.12 105.18) (end 83.19763 105.18) (width 0.2) (layer "F.Cu") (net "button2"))
 (segment (start 82.12 105.18) (end 83.593402 105.18) (width 0.2) (layer "F.Cu") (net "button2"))
 (segment (start 83.19763 105.18) (end 109.15 79.22763) (width 0.2) (layer "F.Cu") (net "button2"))
 (segment (start 108.197056 41.72) (end 109.04 41.72) (width 0.2) (layer "F.Cu") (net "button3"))
 (segment (start 100.33 85.50763) (end 100.33 49.587056) (width 0.2) (layer "F.Cu") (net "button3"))
 (segment (start 83.19763 102.64) (end 100.33 85.50763) (width 0.2) (layer "F.Cu") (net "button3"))
 (segment (start 100.33 49.587056) (end 108.197056 41.72) (width 0.2) (layer "F.Cu") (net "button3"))
 (segment (start 82.12 102.64) (end 83.19763 102.64) (width 0.2) (layer "F.Cu") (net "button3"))
 (segment (start 54.74 69.2) (end 82.12 96.58) (width 0.2) (layer "F.Cu") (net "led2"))
 (segment (start 82.12 96.58) (end 82.12 97.56) (width 0.2) (layer "F.Cu") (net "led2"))
 (segment (start 54.74 45.2) (end 54.74 67.64) (width 0.2) (layer "F.Cu") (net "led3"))
 (segment (start 54.74 67.64) (end 82.12 95.02) (width 0.2) (layer "F.Cu") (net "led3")))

